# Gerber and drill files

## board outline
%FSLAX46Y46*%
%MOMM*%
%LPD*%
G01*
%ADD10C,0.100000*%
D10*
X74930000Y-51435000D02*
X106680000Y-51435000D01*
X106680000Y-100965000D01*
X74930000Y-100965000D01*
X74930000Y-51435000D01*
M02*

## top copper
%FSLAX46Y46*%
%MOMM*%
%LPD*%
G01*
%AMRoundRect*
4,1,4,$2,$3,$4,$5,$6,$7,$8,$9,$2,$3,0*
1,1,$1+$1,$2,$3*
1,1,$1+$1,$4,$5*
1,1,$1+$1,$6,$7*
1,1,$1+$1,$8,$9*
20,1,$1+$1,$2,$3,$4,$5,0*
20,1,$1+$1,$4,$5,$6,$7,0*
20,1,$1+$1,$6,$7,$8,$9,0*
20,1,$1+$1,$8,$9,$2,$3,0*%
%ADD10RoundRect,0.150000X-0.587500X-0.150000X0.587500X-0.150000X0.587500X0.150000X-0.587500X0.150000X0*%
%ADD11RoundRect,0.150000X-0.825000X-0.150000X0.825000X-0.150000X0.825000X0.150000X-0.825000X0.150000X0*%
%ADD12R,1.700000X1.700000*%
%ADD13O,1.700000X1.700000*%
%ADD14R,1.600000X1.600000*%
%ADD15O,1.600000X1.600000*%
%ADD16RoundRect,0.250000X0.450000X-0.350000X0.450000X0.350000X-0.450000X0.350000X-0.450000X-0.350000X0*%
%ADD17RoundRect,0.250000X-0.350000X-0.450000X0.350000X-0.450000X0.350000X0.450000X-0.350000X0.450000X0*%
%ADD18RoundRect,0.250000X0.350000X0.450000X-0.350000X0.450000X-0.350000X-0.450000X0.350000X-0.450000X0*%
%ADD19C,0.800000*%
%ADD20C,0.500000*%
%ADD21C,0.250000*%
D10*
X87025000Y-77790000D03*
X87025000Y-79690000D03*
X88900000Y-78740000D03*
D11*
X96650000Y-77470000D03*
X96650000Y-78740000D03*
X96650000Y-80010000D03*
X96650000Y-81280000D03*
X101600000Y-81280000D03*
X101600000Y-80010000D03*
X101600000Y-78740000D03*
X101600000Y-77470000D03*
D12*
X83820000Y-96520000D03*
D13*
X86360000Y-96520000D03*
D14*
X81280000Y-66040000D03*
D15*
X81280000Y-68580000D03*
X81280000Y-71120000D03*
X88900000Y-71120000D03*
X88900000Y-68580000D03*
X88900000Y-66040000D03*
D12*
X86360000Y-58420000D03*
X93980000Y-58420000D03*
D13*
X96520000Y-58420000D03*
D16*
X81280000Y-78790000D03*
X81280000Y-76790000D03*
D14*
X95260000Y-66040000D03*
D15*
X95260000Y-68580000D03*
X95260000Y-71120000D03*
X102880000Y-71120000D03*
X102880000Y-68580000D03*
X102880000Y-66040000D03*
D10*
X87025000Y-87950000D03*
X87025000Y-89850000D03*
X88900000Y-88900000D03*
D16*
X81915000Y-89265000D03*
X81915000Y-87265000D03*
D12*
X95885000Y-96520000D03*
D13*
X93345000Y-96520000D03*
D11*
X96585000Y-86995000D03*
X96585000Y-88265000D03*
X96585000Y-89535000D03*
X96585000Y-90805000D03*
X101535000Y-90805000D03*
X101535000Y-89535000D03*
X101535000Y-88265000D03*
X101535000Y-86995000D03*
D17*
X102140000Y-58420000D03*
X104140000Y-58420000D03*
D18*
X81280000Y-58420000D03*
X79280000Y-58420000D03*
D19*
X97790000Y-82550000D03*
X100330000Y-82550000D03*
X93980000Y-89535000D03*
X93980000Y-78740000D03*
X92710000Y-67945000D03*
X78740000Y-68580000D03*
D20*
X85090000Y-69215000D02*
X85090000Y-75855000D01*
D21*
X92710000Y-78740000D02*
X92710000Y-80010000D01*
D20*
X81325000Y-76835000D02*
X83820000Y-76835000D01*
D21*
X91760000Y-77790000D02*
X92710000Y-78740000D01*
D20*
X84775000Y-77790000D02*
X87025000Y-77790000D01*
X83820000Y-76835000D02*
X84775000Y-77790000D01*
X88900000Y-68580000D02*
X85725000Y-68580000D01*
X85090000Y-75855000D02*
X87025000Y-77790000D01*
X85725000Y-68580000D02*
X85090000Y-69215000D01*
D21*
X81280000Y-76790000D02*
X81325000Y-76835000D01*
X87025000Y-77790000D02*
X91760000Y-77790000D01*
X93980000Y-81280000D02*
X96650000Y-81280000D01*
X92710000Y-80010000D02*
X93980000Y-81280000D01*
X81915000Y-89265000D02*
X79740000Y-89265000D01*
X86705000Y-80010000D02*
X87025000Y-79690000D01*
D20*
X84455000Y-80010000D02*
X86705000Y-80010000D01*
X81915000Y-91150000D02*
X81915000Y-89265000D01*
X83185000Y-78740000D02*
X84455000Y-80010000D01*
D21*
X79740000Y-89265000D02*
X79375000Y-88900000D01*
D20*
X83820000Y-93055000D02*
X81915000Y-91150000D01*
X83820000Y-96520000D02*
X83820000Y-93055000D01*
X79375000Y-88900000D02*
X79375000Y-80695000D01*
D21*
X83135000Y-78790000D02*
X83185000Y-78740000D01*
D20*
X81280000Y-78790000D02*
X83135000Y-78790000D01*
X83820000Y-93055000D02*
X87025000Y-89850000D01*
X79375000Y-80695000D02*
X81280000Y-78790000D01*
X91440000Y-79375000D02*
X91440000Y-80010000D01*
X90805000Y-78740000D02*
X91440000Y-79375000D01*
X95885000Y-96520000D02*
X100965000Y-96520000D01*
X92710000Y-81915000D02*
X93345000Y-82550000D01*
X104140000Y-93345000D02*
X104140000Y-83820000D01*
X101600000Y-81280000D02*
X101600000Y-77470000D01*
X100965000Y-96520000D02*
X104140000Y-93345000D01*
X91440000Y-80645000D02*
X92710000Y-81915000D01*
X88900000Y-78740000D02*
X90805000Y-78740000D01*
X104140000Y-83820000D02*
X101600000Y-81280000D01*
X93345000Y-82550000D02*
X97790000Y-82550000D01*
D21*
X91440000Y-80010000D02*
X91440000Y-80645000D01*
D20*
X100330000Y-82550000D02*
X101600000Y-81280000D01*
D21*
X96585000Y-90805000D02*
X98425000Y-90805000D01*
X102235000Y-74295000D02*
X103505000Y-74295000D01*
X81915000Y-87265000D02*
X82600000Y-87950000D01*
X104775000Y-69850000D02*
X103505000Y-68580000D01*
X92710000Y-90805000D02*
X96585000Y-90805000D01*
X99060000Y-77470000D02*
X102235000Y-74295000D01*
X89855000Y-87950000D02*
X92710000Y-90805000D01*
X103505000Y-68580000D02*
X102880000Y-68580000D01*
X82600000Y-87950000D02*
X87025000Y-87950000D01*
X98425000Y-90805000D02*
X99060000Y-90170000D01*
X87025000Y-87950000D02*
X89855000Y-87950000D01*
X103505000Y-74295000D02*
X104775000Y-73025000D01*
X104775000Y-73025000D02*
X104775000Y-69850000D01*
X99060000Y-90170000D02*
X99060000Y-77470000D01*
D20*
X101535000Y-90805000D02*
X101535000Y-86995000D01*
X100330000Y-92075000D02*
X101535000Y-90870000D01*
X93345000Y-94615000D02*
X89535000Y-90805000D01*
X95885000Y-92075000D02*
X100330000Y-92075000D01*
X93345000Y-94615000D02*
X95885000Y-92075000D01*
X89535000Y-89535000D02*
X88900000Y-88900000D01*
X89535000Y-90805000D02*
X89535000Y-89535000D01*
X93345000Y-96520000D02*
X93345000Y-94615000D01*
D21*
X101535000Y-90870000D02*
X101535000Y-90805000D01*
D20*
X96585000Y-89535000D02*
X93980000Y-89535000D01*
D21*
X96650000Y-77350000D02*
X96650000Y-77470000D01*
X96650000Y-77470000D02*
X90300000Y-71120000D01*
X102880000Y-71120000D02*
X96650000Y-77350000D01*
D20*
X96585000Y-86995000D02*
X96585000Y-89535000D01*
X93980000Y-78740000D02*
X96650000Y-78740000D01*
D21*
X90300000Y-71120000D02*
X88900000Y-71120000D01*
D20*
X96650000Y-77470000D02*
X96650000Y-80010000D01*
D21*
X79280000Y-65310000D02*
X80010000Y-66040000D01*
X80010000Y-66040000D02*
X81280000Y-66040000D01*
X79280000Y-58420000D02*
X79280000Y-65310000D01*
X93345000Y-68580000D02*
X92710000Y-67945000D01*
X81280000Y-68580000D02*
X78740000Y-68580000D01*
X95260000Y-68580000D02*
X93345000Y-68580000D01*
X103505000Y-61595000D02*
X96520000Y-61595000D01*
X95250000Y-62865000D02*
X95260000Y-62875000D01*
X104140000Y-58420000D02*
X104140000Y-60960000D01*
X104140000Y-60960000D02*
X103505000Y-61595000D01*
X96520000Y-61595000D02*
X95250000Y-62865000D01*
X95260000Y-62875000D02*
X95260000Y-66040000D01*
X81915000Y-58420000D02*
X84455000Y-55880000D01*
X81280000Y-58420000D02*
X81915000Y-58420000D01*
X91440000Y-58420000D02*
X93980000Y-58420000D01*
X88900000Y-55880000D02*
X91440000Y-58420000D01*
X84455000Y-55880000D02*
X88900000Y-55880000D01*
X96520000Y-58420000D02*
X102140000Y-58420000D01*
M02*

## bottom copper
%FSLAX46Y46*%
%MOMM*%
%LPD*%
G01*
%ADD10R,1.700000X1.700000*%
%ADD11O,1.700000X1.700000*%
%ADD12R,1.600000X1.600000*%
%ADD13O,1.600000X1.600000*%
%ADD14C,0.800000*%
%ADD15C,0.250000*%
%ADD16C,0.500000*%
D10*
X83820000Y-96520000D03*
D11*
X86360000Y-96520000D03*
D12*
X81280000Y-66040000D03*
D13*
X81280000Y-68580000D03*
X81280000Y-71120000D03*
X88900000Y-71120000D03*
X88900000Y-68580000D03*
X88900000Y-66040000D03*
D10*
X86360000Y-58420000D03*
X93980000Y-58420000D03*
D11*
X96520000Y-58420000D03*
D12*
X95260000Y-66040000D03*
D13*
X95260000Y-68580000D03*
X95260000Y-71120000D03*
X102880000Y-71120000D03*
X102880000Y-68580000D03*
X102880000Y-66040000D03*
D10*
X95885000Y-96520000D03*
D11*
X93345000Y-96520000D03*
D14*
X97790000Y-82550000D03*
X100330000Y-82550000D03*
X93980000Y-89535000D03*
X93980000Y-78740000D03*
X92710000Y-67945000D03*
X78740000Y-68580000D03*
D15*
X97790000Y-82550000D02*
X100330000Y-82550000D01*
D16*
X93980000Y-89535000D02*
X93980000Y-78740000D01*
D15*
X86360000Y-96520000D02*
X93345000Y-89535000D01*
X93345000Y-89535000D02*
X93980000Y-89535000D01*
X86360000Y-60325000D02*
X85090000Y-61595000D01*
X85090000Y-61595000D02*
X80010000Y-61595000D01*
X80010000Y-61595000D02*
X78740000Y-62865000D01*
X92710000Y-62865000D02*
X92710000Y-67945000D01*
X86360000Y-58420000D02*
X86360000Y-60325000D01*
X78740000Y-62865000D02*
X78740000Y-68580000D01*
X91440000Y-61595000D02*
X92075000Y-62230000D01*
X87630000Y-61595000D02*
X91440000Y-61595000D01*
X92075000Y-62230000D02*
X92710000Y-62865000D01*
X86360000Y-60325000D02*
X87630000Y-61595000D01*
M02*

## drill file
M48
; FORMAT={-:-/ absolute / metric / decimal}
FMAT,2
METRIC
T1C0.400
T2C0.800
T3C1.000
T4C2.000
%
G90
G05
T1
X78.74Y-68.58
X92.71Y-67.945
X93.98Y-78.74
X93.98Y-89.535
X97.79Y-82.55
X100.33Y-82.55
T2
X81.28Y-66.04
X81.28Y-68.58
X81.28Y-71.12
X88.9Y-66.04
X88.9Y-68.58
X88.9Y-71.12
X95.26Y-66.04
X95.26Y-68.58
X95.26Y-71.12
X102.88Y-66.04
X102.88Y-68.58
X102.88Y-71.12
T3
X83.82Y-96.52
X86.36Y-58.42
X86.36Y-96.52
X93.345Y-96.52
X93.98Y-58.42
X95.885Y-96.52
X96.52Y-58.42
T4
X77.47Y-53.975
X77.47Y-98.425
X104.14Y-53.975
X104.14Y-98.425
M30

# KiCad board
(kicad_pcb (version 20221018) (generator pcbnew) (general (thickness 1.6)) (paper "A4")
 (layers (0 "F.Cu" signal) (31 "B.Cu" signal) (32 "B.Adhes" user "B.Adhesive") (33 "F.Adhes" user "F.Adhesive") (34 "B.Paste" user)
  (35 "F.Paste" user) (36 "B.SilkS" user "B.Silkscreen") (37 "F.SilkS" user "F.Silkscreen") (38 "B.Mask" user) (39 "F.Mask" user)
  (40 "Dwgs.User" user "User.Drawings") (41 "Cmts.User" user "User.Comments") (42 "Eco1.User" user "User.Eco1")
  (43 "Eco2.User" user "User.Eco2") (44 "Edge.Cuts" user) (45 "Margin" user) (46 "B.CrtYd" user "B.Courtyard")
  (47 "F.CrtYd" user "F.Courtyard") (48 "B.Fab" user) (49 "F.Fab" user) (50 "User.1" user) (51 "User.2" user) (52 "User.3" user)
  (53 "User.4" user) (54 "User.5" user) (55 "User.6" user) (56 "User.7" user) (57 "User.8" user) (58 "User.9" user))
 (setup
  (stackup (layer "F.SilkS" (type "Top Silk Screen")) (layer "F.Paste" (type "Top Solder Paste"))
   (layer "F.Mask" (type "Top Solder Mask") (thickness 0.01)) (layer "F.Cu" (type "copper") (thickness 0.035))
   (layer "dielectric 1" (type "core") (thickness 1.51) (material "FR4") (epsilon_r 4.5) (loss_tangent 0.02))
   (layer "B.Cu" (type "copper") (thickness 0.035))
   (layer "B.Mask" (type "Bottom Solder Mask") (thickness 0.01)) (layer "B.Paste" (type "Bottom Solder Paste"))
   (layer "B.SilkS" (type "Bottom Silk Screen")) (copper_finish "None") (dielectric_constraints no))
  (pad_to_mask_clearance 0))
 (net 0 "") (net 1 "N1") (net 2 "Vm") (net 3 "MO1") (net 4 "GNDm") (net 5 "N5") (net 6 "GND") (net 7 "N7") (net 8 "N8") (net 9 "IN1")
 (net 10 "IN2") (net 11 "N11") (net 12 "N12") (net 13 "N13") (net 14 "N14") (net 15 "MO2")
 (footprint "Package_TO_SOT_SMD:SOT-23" (layer "F.Cu") (at 87.9625 78.74)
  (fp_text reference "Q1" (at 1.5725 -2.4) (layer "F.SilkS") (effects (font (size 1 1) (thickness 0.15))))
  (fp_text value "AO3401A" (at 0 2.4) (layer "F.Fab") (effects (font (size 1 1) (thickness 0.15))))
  (pad "1" smd roundrect (at -0.9375 -0.95) (size 1.475 0.6) (layers "F.Cu" "F.Paste" "F.Mask") (roundrect_rratio 0.25) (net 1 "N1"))
  (pad "2" smd roundrect (at -0.9375 0.95) (size 1.475 0.6) (layers "F.Cu" "F.Paste" "F.Mask") (roundrect_rratio 0.25) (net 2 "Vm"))
  (pad "3" smd roundrect (at 0.9375 0) (size 1.475 0.6) (layers "F.Cu" "F.Paste" "F.Mask") (roundrect_rratio 0.25) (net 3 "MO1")))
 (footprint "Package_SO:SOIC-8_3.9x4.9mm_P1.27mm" (layer "F.Cu") (at 99.125 79.375)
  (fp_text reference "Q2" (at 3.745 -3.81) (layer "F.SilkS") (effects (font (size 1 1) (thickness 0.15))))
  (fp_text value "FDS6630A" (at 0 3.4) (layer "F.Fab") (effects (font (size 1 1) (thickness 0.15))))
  (pad "1" smd roundrect (at -2.475 -1.905) (size 1.95 0.6) (layers "F.Cu" "F.Paste" "F.Mask") (roundrect_rratio 0.25) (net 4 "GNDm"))
  (pad "2" smd roundrect (at -2.475 -0.635) (size 1.95 0.6) (layers "F.Cu" "F.Paste" "F.Mask") (roundrect_rratio 0.25) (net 4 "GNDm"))
  (pad "3" smd roundrect (at -2.475 0.635) (size 1.95 0.6) (layers "F.Cu" "F.Paste" "F.Mask") (roundrect_rratio 0.25) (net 4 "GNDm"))
  (pad "4" smd roundrect (at -2.475 1.905) (size 1.95 0.6) (layers "F.Cu" "F.Paste" "F.Mask") (roundrect_rratio 0.25) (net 1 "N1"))
  (pad "5" smd roundrect (at 2.475 1.905) (size 1.95 0.6) (layers "F.Cu" "F.Paste" "F.Mask") (roundrect_rratio 0.25) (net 3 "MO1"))
  (pad "6" smd roundrect (at 2.475 0.635) (size 1.95 0.6) (layers "F.Cu" "F.Paste" "F.Mask") (roundrect_rratio 0.25) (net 3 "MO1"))
  (pad "7" smd roundrect (at 2.475 -0.635) (size 1.95 0.6) (layers "F.Cu" "F.Paste" "F.Mask") (roundrect_rratio 0.25) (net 3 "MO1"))
  (pad "8" smd roundrect (at 2.475 -1.905) (size 1.95 0.6) (layers "F.Cu" "F.Paste" "F.Mask") (roundrect_rratio 0.25) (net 3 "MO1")))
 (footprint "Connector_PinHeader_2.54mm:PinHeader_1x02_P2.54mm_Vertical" (layer "F.Cu") (at 83.82 96.52 90)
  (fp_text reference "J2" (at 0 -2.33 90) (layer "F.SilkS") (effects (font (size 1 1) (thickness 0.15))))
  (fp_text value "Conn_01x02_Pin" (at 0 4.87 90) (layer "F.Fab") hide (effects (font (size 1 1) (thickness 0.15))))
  (pad "1" thru_hole rect (at 0 0 90) (size 1.7 1.7) (drill 1) (layers "*.Cu" "*.Mask") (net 2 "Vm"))
  (pad "2" thru_hole oval (at 0 2.54 90) (size 1.7 1.7) (drill 1) (layers "*.Cu" "*.Mask") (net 4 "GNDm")))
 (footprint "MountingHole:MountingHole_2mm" (layer "F.Cu") (at 104.14 53.975)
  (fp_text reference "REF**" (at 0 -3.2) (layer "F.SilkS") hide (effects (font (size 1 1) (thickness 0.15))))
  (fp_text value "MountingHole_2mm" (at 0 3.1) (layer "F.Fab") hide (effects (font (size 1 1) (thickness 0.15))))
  (pad "" np_thru_hole circle (at 0 0) (size 2 2) (drill 2) (layers "*.Cu" "*.Mask")))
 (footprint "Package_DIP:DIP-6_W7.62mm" (layer "F.Cu") (at 81.28 66.04)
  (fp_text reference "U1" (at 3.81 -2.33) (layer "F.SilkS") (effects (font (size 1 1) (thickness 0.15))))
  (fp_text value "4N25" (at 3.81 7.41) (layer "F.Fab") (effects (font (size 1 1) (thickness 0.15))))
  (pad "1" thru_hole rect (at 0 0) (size 1.6 1.6) (drill 0.8) (layers "*.Cu" "*.Mask") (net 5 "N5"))
  (pad "2" thru_hole oval (at 0 2.54) (size 1.6 1.6) (drill 0.8) (layers "*.Cu" "*.Mask") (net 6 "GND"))
  (pad "3" thru_hole oval (at 0 5.08) (size 1.6 1.6) (drill 0.8) (layers "*.Cu" "*.Mask") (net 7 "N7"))
  (pad "4" thru_hole oval (at 7.62 5.08) (size 1.6 1.6) (drill 0.8) (layers "*.Cu" "*.Mask") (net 4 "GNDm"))
  (pad "5" thru_hole oval (at 7.62 2.54) (size 1.6 1.6) (drill 0.8) (layers "*.Cu" "*.Mask") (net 1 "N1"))
  (pad "6" thru_hole oval (at 7.62 0) (size 1.6 1.6) (drill 0.8) (layers "*.Cu" "*.Mask") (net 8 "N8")))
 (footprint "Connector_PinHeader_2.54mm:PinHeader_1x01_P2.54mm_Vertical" (layer "F.Cu") (at 86.36 58.42)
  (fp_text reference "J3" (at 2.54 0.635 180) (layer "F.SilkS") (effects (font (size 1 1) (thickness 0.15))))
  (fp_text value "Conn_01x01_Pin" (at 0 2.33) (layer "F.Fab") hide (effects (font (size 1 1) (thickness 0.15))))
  (pad "1" thru_hole rect (at 0 0) (size 1.7 1.7) (drill 1) (layers "*.Cu" "*.Mask") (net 6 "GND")))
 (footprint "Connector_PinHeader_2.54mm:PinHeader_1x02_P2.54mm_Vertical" (layer "F.Cu") (at 93.98 58.42 90)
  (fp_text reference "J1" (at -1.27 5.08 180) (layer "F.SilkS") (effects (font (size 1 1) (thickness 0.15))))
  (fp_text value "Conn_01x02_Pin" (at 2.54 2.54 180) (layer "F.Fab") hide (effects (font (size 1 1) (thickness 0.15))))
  (pad "1" thru_hole rect (at 0 0 90) (size 1.7 1.7) (drill 1) (layers "*.Cu" "*.Mask") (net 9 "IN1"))
  (pad "2" thru_hole oval (at 0 2.54 90) (size 1.7 1.7) (drill 1) (layers "*.Cu" "*.Mask") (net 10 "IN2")))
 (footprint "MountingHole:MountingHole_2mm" (layer "F.Cu") (at 77.47 98.425)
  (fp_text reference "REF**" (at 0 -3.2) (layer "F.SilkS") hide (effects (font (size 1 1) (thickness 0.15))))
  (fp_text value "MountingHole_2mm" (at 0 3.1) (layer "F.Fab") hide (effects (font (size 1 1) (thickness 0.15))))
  (pad "" np_thru_hole circle (at 0 0) (size 2 2) (drill 2) (layers "*.Cu" "*.Mask")))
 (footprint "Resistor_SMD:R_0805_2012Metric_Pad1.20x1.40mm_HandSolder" (layer "F.Cu") (at 81.28 77.79 90)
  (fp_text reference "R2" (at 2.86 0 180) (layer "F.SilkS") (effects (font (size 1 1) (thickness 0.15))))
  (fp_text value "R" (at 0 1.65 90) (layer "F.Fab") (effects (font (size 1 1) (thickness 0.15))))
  (pad "1" smd roundrect (at -1 0 90) (size 1.2 1.4) (layers "F.Cu" "F.Paste" "F.Mask") (roundrect_rratio 0.208333) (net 2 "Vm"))
  (pad "2" smd roundrect (at 1 0 90) (size 1.2 1.4) (layers "F.Cu" "F.Paste" "F.Mask") (roundrect_rratio 0.208333) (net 1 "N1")))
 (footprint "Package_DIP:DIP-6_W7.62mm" (layer "F.Cu") (at 95.26 66.04)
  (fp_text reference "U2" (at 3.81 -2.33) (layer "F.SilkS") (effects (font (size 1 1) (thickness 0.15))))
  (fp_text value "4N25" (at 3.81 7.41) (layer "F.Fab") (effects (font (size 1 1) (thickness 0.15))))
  (pad "1" thru_hole rect (at 0 0) (size 1.6 1.6) (drill 0.8) (layers "*.Cu" "*.Mask") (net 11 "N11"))
  (pad "2" thru_hole oval (at 0 2.54) (size 1.6 1.6) (drill 0.8) (layers "*.Cu" "*.Mask") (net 6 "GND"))
  (pad "3" thru_hole oval (at 0 5.08) (size 1.6 1.6) (drill 0.8) (layers "*.Cu" "*.Mask") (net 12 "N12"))
  (pad "4" thru_hole oval (at 7.62 5.08) (size 1.6 1.6) (drill 0.8) (layers "*.Cu" "*.Mask") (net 4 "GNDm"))
  (pad "5" thru_hole oval (at 7.62 2.54) (size 1.6 1.6) (drill 0.8) (layers "*.Cu" "*.Mask") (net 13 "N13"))
  (pad "6" thru_hole oval (at 7.62 0) (size 1.6 1.6) (drill 0.8) (layers "*.Cu" "*.Mask") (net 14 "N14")))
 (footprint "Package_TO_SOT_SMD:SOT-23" (layer "F.Cu") (at 87.9625 88.9)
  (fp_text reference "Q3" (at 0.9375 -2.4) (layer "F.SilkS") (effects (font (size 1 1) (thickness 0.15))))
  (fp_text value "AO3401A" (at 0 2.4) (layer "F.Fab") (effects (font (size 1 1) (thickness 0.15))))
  (pad "1" smd roundrect (at -0.9375 -0.95) (size 1.475 0.6) (layers "F.Cu" "F.Paste" "F.Mask") (roundrect_rratio 0.25) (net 13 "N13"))
  (pad "2" smd roundrect (at -0.9375 0.95) (size 1.475 0.6) (layers "F.Cu" "F.Paste" "F.Mask") (roundrect_rratio 0.25) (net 2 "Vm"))
  (pad "3" smd roundrect (at 0.9375 0) (size 1.475 0.6) (layers "F.Cu" "F.Paste" "F.Mask") (roundrect_rratio 0.25) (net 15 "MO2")))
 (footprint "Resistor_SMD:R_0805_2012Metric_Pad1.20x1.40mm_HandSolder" (layer "F.Cu") (at 81.915 88.265 90)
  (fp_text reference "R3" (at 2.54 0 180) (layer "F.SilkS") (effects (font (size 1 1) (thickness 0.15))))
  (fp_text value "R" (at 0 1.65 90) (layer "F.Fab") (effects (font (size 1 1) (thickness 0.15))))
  (pad "1" smd roundrect (at -1 0 90) (size 1.2 1.4) (layers "F.Cu" "F.Paste" "F.Mask") (roundrect_rratio 0.208333) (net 2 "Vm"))
  (pad "2" smd roundrect (at 1 0 90) (size 1.2 1.4) (layers "F.Cu" "F.Paste" "F.Mask") (roundrect_rratio 0.208333) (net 13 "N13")))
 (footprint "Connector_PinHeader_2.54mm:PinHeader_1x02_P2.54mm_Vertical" (layer "F.Cu") (at 95.885 96.52 -90)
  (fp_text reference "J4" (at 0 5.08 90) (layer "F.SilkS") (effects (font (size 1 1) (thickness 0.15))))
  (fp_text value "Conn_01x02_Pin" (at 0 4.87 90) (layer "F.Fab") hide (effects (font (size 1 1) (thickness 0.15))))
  (pad "1" thru_hole rect (at 0 0 270) (size 1.7 1.7) (drill 1) (layers "*.Cu" "*.Mask") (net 3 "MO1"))
  (pad "2" thru_hole oval (at 0 2.54 270) (size 1.7 1.7) (drill 1) (layers "*.Cu" "*.Mask") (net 15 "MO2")))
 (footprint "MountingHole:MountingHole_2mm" (layer "F.Cu") (at 77.47 53.975)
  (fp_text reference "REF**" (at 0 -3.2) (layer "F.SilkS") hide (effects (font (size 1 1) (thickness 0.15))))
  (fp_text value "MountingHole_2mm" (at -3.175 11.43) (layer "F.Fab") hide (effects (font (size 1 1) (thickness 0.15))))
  (pad "" np_thru_hole circle (at 0 0) (size 2 2) (drill 2) (layers "*.Cu" "*.Mask")))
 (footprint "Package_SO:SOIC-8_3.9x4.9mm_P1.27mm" (layer "F.Cu") (at 99.06 88.9)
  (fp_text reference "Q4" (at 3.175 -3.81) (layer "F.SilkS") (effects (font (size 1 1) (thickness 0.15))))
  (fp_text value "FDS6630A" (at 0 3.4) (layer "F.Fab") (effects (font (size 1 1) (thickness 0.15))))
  (pad "1" smd roundrect (at -2.475 -1.905) (size 1.95 0.6) (layers "F.Cu" "F.Paste" "F.Mask") (roundrect_rratio 0.25) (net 4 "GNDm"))
  (pad "2" smd roundrect (at -2.475 -0.635) (size 1.95 0.6) (layers "F.Cu" "F.Paste" "F.Mask") (roundrect_rratio 0.25) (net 4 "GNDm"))
  (pad "3" smd roundrect (at -2.475 0.635) (size 1.95 0.6) (layers "F.Cu" "F.Paste" "F.Mask") (roundrect_rratio 0.25) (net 4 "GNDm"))
  (pad "4" smd roundrect (at -2.475 1.905) (size 1.95 0.6) (layers "F.Cu" "F.Paste" "F.Mask") (roundrect_rratio 0.25) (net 13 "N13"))
  (pad "5" smd roundrect (at 2.475 1.905) (size 1.95 0.6) (layers "F.Cu" "F.Paste" "F.Mask") (roundrect_rratio 0.25) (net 15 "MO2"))
  (pad "6" smd roundrect (at 2.475 0.635) (size 1.95 0.6) (layers "F.Cu" "F.Paste" "F.Mask") (roundrect_rratio 0.25) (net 15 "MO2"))
  (pad "7" smd roundrect (at 2.475 -0.635) (size 1.95 0.6) (layers "F.Cu" "F.Paste" "F.Mask") (roundrect_rratio 0.25) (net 15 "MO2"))
  (pad "8" smd roundrect (at 2.475 -1.905) (size 1.95 0.6) (layers "F.Cu" "F.Paste" "F.Mask") (roundrect_rratio 0.25) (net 15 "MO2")))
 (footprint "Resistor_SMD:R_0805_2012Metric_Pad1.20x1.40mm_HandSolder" (layer "F.Cu") (at 103.14 58.42)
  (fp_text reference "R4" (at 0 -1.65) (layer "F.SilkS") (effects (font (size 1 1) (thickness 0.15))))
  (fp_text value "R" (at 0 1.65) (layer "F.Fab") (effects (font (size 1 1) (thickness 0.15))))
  (pad "1" smd roundrect (at -1 0) (size 1.2 1.4) (layers "F.Cu" "F.Paste" "F.Mask") (roundrect_rratio 0.208333) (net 10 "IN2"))
  (pad "2" smd roundrect (at 1 0) (size 1.2 1.4) (layers "F.Cu" "F.Paste" "F.Mask") (roundrect_rratio 0.208333) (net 11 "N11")))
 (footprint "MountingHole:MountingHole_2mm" (layer "F.Cu") (at 104.14 98.425)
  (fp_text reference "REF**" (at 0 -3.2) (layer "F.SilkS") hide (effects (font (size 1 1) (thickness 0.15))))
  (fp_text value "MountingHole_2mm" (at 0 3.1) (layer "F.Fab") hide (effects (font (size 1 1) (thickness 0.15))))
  (pad "" np_thru_hole circle (at 0 0) (size 2 2) (drill 2) (layers "*.Cu" "*.Mask")))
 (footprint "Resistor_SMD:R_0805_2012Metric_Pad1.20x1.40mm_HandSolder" (layer "F.Cu") (at 80.28 58.42 180)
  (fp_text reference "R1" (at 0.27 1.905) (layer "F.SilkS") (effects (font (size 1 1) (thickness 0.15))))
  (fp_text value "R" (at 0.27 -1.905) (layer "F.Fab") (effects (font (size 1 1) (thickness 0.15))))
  (pad "1" smd roundrect (at -1 0 180) (size 1.2 1.4) (layers "F.Cu" "F.Paste" "F.Mask") (roundrect_rratio 0.208333) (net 9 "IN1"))
  (pad "2" smd roundrect (at 1 0 180) (size 1.2 1.4) (layers "F.Cu" "F.Paste" "F.Mask") (roundrect_rratio 0.208333) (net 5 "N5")))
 (gr_rect (start 74.93 51.435) (end 106.68 100.965) (stroke (width 0.1) (type default)) (fill none) (layer "Edge.Cuts"))
 (segment (start 85.09 69.215) (end 85.09 75.855) (width 0.5) (layer "F.Cu") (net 1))
 (segment (start 92.71 78.74) (end 92.71 80.01) (width 0.25) (layer "F.Cu") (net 1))
 (segment (start 81.325 76.835) (end 83.82 76.835) (width 0.5) (layer "F.Cu") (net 1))
 (segment (start 91.76 77.79) (end 92.71 78.74) (width 0.25) (layer "F.Cu") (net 1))
 (segment (start 84.775 77.79) (end 87.025 77.79) (width 0.5) (layer "F.Cu") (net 1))
 (segment (start 83.82 76.835) (end 84.775 77.79) (width 0.5) (layer "F.Cu") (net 1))
 (segment (start 88.9 68.58) (end 85.725 68.58) (width 0.5) (layer "F.Cu") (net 1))
 (segment (start 85.09 75.855) (end 87.025 77.79) (width 0.5) (layer "F.Cu") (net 1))
 (segment (start 85.725 68.58) (end 85.09 69.215) (width 0.5) (layer "F.Cu") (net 1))
 (segment (start 81.28 76.79) (end 81.325 76.835) (width 0.25) (layer "F.Cu") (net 1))
 (segment (start 87.025 77.79) (end 91.76 77.79) (width 0.25) (layer "F.Cu") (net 1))
 (segment (start 93.98 81.28) (end 96.65 81.28) (width 0.25) (layer "F.Cu") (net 1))
 (segment (start 92.71 80.01) (end 93.98 81.28) (width 0.25) (layer "F.Cu") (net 1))
 (segment (start 81.915 89.265) (end 79.74 89.265) (width 0.25) (layer "F.Cu") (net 2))
 (segment (start 86.705 80.01) (end 87.025 79.69) (width 0.25) (layer "F.Cu") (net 2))
 (segment (start 84.455 80.01) (end 86.705 80.01) (width 0.5) (layer "F.Cu") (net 2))
 (segment (start 81.915 91.15) (end 81.915 89.265) (width 0.5) (layer "F.Cu") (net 2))
 (segment (start 83.185 78.74) (end 84.455 80.01) (width 0.5) (layer "F.Cu") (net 2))
 (segment (start 79.74 89.265) (end 79.375 88.9) (width 0.25) (layer "F.Cu") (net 2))
 (segment (start 83.82 93.055) (end 81.915 91.15) (width 0.5) (layer "F.Cu") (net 2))
 (segment (start 83.82 96.52) (end 83.82 93.055) (width 0.5) (layer "F.Cu") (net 2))
 (segment (start 79.375 88.9) (end 79.375 80.695) (width 0.5) (layer "F.Cu") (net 2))
 (segment (start 83.135 78.79) (end 83.185 78.74) (width 0.25) (layer "F.Cu") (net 2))
 (segment (start 81.28 78.79) (end 83.135 78.79) (width 0.5) (layer "F.Cu") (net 2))
 (segment (start 83.82 93.055) (end 87.025 89.85) (width 0.5) (layer "F.Cu") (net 2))
 (segment (start 79.375 80.695) (end 81.28 78.79) (width 0.5) (layer "F.Cu") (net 2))
 (segment (start 91.44 79.375) (end 91.44 80.01) (width 0.5) (layer "F.Cu") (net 3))
 (segment (start 90.805 78.74) (end 91.44 79.375) (width 0.5) (layer "F.Cu") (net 3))
 (segment (start 95.885 96.52) (end 100.965 96.52) (width 0.5) (layer "F.Cu") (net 3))
 (segment (start 92.71 81.915) (end 93.345 82.55) (width 0.5) (layer "F.Cu") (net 3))
 (segment (start 104.14 93.345) (end 104.14 83.82) (width 0.5) (layer "F.Cu") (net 3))
 (segment (start 101.6 81.28) (end 101.6 77.47) (width 0.5) (layer "F.Cu") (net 3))
 (segment (start 100.965 96.52) (end 104.14 93.345) (width 0.5) (layer "F.Cu") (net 3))
 (segment (start 91.44 80.645) (end 92.71 81.915) (width 0.5) (layer "F.Cu") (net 3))
 (segment (start 88.9 78.74) (end 90.805 78.74) (width 0.5) (layer "F.Cu") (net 3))
 (segment (start 104.14 83.82) (end 101.6 81.28) (width 0.5) (layer "F.Cu") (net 3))
 (segment (start 93.345 82.55) (end 97.79 82.55) (width 0.5) (layer "F.Cu") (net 3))
 (segment (start 91.44 80.01) (end 91.44 80.645) (width 0.25) (layer "F.Cu") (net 3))
 (segment (start 100.33 82.55) (end 101.6 81.28) (width 0.5) (layer "F.Cu") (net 3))
 (via (at 97.79 82.55) (size 0.8) (drill 0.4) (layers "F.Cu" "B.Cu") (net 3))
 (via (at 100.33 82.55) (size 0.8) (drill 0.4) (layers "F.Cu" "B.Cu") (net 3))
 (segment (start 97.79 82.55) (end 100.33 82.55) (width 0.25) (layer "B.Cu") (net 3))
 (segment (start 96.585 90.805) (end 98.425 90.805) (width 0.25) (layer "F.Cu") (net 13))
 (segment (start 102.235 74.295) (end 103.505 74.295) (width 0.25) (layer "F.Cu") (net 13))
 (segment (start 81.915 87.265) (end 82.6 87.95) (width 0.25) (layer "F.Cu") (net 13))
 (segment (start 104.775 69.85) (end 103.505 68.58) (width 0.25) (layer "F.Cu") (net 13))
 (segment (start 92.71 90.805) (end 96.585 90.805) (width 0.25) (layer "F.Cu") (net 13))
 (segment (start 99.06 77.47) (end 102.235 74.295) (width 0.25) (layer "F.Cu") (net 13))
 (segment (start 89.855 87.95) (end 92.71 90.805) (width 0.25) (layer "F.Cu") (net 13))
 (segment (start 103.505 68.58) (end 102.88 68.58) (width 0.25) (layer "F.Cu") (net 13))
 (segment (start 82.6 87.95) (end 87.025 87.95) (width 0.25) (layer "F.Cu") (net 13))
 (segment (start 98.425 90.805) (end 99.06 90.17) (width 0.25) (layer "F.Cu") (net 13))
 (segment (start 87.025 87.95) (end 89.855 87.95) (width 0.25) (layer "F.Cu") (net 13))
 (segment (start 103.505 74.295) (end 104.775 73.025) (width 0.25) (layer "F.Cu") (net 13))
 (segment (start 104.775 73.025) (end 104.775 69.85) (width 0.25) (layer "F.Cu") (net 13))
 (segment (start 99.06 90.17) (end 99.06 77.47) (width 0.25) (layer "F.Cu") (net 13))
 (segment (start 101.535 90.805) (end 101.535 86.995) (width 0.5) (layer "F.Cu") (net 15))
 (segment (start 100.33 92.075) (end 101.535 90.87) (width 0.5) (layer "F.Cu") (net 15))
 (segment (start 93.345 94.615) (end 89.535 90.805) (width 0.5) (layer "F.Cu") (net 15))
 (segment (start 95.885 92.075) (end 100.33 92.075) (width 0.5) (layer "F.Cu") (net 15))
 (segment (start 93.345 94.615) (end 95.885 92.075) (width 0.5) (layer "F.Cu") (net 15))
 (segment (start 89.535 89.535) (end 88.9 88.9) (width 0.5) (layer "F.Cu") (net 15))
 (segment (start 89.535 90.805) (end 89.535 89.535) (width 0.5) (layer "F.Cu") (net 15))
 (segment (start 93.345 96.52) (end 93.345 94.615) (width 0.5) (layer "F.Cu") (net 15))
 (segment (start 101.535 90.87) (end 101.535 90.805) (width 0.25) (layer "F.Cu") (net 15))
 (segment (start 96.585 89.535) (end 93.98 89.535) (width 0.5) (layer "F.Cu") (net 4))
 (segment (start 96.65 77.35) (end 96.65 77.47) (width 0.25) (layer "F.Cu") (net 4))
 (segment (start 96.65 77.47) (end 90.3 71.12) (width 0.25) (layer "F.Cu") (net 4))
 (segment (start 102.88 71.12) (end 96.65 77.35) (width 0.25) (layer "F.Cu") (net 4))
 (segment (start 96.585 86.995) (end 96.585 89.535) (width 0.5) (layer "F.Cu") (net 4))
 (segment (start 93.98 78.74) (end 96.65 78.74) (width 0.5) (layer "F.Cu") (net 4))
 (segment (start 90.3 71.12) (end 88.9 71.12) (width 0.25) (layer "F.Cu") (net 4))
 (segment (start 96.65 77.47) (end 96.65 80.01) (width 0.5) (layer "F.Cu") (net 4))
 (via (at 93.98 89.535) (size 0.8) (drill 0.4) (layers "F.Cu" "B.Cu") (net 4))
 (via (at 93.98 78.74) (size 0.8) (drill 0.4) (layers "F.Cu" "B.Cu") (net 4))
 (segment (start 93.98 89.535) (end 93.98 78.74) (width 0.5) (layer "B.Cu") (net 4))
 (segment (start 86.36 96.52) (end 93.345 89.535) (width 0.25) (layer "B.Cu") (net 4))
 (segment (start 93.345 89.535) (end 93.98 89.535) (width 0.25) (layer "B.Cu") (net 4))
 (segment (start 79.28 65.31) (end 80.01 66.04) (width 0.25) (layer "F.Cu") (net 5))
 (segment (start 80.01 66.04) (end 81.28 66.04) (width 0.25) (layer "F.Cu") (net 5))
 (segment (start 79.28 58.42) (end 79.28 65.31) (width 0.25) (layer "F.Cu") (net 5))
 (segment (start 93.345 68.58) (end 92.71 67.945) (width 0.25) (layer "F.Cu") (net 6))
 (segment (start 81.28 68.58) (end 78.74 68.58) (width 0.25) (layer "F.Cu") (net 6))
 (segment (start 95.26 68.58) (end 93.345 68.58) (width 0.25) (layer "F.Cu") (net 6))
 (via (at 92.71 67.945) (size 0.8) (drill 0.4) (layers "F.Cu" "B.Cu") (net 6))
 (via (at 78.74 68.58) (size 0.8) (drill 0.4) (layers "F.Cu" "B.Cu") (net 6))
 (segment (start 86.36 60.325) (end 85.09 61.595) (width 0.25) (layer "B.Cu") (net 6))
 (segment (start 85.09 61.595) (end 80.01 61.595) (width 0.25) (layer "B.Cu") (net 6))
 (segment (start 80.01 61.595) (end 78.74 62.865) (width 0.25) (layer "B.Cu") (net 6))
 (segment (start 92.71 62.865) (end 92.71 67.945) (width 0.25) (layer "B.Cu") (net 6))
 (segment (start 86.36 58.42) (end 86.36 60.325) (width 0.25) (layer "B.Cu") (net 6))
 (segment (start 78.74 62.865) (end 78.74 68.58) (width 0.25) (layer "B.Cu") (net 6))
 (segment (start 91.44 61.595) (end 92.075 62.23) (width 0.25) (layer "B.Cu") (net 6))
 (segment (start 87.63 61.595) (end 91.44 61.595) (width 0.25) (layer "B.Cu") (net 6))
 (segment (start 92.075 62.23) (end 92.71 62.865) (width 0.25) (layer "B.Cu") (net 6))
 (segment (start 86.36 60.325) (end 87.63 61.595) (width 0.25) (layer "B.Cu") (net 6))
 (segment (start 103.505 61.595) (end 96.52 61.595) (width 0.25) (layer "F.Cu") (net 11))
 (segment (start 95.25 62.865) (end 95.26 62.875) (width 0.25) (layer "F.Cu") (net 11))
 (segment (start 104.14 58.42) (end 104.14 60.96) (width 0.25) (layer "F.Cu") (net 11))
 (segment (start 104.14 60.96) (end 103.505 61.595) (width 0.25) (layer "F.Cu") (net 11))
 (segment (start 96.52 61.595) (end 95.25 62.865) (width 0.25) (layer "F.Cu") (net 11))
 (segment (start 95.26 62.875) (end 95.26 66.04) (width 0.25) (layer "F.Cu") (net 11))
 (segment (start 81.915 58.42) (end 84.455 55.88) (width 0.25) (layer "F.Cu") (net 9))
 (segment (start 81.28 58.42) (end 81.915 58.42) (width 0.25) (layer "F.Cu") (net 9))
 (segment (start 91.44 58.42) (end 93.98 58.42) (width 0.25) (layer "F.Cu") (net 9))
 (segment (start 88.9 55.88) (end 91.44 58.42) (width 0.25) (layer "F.Cu") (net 9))
 (segment (start 84.455 55.88) (end 88.9 55.88) (width 0.25) (layer "F.Cu") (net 9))
 (segment (start 96.52 58.42) (end 102.14 58.42) (width 0.25) (layer "F.Cu") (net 10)))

